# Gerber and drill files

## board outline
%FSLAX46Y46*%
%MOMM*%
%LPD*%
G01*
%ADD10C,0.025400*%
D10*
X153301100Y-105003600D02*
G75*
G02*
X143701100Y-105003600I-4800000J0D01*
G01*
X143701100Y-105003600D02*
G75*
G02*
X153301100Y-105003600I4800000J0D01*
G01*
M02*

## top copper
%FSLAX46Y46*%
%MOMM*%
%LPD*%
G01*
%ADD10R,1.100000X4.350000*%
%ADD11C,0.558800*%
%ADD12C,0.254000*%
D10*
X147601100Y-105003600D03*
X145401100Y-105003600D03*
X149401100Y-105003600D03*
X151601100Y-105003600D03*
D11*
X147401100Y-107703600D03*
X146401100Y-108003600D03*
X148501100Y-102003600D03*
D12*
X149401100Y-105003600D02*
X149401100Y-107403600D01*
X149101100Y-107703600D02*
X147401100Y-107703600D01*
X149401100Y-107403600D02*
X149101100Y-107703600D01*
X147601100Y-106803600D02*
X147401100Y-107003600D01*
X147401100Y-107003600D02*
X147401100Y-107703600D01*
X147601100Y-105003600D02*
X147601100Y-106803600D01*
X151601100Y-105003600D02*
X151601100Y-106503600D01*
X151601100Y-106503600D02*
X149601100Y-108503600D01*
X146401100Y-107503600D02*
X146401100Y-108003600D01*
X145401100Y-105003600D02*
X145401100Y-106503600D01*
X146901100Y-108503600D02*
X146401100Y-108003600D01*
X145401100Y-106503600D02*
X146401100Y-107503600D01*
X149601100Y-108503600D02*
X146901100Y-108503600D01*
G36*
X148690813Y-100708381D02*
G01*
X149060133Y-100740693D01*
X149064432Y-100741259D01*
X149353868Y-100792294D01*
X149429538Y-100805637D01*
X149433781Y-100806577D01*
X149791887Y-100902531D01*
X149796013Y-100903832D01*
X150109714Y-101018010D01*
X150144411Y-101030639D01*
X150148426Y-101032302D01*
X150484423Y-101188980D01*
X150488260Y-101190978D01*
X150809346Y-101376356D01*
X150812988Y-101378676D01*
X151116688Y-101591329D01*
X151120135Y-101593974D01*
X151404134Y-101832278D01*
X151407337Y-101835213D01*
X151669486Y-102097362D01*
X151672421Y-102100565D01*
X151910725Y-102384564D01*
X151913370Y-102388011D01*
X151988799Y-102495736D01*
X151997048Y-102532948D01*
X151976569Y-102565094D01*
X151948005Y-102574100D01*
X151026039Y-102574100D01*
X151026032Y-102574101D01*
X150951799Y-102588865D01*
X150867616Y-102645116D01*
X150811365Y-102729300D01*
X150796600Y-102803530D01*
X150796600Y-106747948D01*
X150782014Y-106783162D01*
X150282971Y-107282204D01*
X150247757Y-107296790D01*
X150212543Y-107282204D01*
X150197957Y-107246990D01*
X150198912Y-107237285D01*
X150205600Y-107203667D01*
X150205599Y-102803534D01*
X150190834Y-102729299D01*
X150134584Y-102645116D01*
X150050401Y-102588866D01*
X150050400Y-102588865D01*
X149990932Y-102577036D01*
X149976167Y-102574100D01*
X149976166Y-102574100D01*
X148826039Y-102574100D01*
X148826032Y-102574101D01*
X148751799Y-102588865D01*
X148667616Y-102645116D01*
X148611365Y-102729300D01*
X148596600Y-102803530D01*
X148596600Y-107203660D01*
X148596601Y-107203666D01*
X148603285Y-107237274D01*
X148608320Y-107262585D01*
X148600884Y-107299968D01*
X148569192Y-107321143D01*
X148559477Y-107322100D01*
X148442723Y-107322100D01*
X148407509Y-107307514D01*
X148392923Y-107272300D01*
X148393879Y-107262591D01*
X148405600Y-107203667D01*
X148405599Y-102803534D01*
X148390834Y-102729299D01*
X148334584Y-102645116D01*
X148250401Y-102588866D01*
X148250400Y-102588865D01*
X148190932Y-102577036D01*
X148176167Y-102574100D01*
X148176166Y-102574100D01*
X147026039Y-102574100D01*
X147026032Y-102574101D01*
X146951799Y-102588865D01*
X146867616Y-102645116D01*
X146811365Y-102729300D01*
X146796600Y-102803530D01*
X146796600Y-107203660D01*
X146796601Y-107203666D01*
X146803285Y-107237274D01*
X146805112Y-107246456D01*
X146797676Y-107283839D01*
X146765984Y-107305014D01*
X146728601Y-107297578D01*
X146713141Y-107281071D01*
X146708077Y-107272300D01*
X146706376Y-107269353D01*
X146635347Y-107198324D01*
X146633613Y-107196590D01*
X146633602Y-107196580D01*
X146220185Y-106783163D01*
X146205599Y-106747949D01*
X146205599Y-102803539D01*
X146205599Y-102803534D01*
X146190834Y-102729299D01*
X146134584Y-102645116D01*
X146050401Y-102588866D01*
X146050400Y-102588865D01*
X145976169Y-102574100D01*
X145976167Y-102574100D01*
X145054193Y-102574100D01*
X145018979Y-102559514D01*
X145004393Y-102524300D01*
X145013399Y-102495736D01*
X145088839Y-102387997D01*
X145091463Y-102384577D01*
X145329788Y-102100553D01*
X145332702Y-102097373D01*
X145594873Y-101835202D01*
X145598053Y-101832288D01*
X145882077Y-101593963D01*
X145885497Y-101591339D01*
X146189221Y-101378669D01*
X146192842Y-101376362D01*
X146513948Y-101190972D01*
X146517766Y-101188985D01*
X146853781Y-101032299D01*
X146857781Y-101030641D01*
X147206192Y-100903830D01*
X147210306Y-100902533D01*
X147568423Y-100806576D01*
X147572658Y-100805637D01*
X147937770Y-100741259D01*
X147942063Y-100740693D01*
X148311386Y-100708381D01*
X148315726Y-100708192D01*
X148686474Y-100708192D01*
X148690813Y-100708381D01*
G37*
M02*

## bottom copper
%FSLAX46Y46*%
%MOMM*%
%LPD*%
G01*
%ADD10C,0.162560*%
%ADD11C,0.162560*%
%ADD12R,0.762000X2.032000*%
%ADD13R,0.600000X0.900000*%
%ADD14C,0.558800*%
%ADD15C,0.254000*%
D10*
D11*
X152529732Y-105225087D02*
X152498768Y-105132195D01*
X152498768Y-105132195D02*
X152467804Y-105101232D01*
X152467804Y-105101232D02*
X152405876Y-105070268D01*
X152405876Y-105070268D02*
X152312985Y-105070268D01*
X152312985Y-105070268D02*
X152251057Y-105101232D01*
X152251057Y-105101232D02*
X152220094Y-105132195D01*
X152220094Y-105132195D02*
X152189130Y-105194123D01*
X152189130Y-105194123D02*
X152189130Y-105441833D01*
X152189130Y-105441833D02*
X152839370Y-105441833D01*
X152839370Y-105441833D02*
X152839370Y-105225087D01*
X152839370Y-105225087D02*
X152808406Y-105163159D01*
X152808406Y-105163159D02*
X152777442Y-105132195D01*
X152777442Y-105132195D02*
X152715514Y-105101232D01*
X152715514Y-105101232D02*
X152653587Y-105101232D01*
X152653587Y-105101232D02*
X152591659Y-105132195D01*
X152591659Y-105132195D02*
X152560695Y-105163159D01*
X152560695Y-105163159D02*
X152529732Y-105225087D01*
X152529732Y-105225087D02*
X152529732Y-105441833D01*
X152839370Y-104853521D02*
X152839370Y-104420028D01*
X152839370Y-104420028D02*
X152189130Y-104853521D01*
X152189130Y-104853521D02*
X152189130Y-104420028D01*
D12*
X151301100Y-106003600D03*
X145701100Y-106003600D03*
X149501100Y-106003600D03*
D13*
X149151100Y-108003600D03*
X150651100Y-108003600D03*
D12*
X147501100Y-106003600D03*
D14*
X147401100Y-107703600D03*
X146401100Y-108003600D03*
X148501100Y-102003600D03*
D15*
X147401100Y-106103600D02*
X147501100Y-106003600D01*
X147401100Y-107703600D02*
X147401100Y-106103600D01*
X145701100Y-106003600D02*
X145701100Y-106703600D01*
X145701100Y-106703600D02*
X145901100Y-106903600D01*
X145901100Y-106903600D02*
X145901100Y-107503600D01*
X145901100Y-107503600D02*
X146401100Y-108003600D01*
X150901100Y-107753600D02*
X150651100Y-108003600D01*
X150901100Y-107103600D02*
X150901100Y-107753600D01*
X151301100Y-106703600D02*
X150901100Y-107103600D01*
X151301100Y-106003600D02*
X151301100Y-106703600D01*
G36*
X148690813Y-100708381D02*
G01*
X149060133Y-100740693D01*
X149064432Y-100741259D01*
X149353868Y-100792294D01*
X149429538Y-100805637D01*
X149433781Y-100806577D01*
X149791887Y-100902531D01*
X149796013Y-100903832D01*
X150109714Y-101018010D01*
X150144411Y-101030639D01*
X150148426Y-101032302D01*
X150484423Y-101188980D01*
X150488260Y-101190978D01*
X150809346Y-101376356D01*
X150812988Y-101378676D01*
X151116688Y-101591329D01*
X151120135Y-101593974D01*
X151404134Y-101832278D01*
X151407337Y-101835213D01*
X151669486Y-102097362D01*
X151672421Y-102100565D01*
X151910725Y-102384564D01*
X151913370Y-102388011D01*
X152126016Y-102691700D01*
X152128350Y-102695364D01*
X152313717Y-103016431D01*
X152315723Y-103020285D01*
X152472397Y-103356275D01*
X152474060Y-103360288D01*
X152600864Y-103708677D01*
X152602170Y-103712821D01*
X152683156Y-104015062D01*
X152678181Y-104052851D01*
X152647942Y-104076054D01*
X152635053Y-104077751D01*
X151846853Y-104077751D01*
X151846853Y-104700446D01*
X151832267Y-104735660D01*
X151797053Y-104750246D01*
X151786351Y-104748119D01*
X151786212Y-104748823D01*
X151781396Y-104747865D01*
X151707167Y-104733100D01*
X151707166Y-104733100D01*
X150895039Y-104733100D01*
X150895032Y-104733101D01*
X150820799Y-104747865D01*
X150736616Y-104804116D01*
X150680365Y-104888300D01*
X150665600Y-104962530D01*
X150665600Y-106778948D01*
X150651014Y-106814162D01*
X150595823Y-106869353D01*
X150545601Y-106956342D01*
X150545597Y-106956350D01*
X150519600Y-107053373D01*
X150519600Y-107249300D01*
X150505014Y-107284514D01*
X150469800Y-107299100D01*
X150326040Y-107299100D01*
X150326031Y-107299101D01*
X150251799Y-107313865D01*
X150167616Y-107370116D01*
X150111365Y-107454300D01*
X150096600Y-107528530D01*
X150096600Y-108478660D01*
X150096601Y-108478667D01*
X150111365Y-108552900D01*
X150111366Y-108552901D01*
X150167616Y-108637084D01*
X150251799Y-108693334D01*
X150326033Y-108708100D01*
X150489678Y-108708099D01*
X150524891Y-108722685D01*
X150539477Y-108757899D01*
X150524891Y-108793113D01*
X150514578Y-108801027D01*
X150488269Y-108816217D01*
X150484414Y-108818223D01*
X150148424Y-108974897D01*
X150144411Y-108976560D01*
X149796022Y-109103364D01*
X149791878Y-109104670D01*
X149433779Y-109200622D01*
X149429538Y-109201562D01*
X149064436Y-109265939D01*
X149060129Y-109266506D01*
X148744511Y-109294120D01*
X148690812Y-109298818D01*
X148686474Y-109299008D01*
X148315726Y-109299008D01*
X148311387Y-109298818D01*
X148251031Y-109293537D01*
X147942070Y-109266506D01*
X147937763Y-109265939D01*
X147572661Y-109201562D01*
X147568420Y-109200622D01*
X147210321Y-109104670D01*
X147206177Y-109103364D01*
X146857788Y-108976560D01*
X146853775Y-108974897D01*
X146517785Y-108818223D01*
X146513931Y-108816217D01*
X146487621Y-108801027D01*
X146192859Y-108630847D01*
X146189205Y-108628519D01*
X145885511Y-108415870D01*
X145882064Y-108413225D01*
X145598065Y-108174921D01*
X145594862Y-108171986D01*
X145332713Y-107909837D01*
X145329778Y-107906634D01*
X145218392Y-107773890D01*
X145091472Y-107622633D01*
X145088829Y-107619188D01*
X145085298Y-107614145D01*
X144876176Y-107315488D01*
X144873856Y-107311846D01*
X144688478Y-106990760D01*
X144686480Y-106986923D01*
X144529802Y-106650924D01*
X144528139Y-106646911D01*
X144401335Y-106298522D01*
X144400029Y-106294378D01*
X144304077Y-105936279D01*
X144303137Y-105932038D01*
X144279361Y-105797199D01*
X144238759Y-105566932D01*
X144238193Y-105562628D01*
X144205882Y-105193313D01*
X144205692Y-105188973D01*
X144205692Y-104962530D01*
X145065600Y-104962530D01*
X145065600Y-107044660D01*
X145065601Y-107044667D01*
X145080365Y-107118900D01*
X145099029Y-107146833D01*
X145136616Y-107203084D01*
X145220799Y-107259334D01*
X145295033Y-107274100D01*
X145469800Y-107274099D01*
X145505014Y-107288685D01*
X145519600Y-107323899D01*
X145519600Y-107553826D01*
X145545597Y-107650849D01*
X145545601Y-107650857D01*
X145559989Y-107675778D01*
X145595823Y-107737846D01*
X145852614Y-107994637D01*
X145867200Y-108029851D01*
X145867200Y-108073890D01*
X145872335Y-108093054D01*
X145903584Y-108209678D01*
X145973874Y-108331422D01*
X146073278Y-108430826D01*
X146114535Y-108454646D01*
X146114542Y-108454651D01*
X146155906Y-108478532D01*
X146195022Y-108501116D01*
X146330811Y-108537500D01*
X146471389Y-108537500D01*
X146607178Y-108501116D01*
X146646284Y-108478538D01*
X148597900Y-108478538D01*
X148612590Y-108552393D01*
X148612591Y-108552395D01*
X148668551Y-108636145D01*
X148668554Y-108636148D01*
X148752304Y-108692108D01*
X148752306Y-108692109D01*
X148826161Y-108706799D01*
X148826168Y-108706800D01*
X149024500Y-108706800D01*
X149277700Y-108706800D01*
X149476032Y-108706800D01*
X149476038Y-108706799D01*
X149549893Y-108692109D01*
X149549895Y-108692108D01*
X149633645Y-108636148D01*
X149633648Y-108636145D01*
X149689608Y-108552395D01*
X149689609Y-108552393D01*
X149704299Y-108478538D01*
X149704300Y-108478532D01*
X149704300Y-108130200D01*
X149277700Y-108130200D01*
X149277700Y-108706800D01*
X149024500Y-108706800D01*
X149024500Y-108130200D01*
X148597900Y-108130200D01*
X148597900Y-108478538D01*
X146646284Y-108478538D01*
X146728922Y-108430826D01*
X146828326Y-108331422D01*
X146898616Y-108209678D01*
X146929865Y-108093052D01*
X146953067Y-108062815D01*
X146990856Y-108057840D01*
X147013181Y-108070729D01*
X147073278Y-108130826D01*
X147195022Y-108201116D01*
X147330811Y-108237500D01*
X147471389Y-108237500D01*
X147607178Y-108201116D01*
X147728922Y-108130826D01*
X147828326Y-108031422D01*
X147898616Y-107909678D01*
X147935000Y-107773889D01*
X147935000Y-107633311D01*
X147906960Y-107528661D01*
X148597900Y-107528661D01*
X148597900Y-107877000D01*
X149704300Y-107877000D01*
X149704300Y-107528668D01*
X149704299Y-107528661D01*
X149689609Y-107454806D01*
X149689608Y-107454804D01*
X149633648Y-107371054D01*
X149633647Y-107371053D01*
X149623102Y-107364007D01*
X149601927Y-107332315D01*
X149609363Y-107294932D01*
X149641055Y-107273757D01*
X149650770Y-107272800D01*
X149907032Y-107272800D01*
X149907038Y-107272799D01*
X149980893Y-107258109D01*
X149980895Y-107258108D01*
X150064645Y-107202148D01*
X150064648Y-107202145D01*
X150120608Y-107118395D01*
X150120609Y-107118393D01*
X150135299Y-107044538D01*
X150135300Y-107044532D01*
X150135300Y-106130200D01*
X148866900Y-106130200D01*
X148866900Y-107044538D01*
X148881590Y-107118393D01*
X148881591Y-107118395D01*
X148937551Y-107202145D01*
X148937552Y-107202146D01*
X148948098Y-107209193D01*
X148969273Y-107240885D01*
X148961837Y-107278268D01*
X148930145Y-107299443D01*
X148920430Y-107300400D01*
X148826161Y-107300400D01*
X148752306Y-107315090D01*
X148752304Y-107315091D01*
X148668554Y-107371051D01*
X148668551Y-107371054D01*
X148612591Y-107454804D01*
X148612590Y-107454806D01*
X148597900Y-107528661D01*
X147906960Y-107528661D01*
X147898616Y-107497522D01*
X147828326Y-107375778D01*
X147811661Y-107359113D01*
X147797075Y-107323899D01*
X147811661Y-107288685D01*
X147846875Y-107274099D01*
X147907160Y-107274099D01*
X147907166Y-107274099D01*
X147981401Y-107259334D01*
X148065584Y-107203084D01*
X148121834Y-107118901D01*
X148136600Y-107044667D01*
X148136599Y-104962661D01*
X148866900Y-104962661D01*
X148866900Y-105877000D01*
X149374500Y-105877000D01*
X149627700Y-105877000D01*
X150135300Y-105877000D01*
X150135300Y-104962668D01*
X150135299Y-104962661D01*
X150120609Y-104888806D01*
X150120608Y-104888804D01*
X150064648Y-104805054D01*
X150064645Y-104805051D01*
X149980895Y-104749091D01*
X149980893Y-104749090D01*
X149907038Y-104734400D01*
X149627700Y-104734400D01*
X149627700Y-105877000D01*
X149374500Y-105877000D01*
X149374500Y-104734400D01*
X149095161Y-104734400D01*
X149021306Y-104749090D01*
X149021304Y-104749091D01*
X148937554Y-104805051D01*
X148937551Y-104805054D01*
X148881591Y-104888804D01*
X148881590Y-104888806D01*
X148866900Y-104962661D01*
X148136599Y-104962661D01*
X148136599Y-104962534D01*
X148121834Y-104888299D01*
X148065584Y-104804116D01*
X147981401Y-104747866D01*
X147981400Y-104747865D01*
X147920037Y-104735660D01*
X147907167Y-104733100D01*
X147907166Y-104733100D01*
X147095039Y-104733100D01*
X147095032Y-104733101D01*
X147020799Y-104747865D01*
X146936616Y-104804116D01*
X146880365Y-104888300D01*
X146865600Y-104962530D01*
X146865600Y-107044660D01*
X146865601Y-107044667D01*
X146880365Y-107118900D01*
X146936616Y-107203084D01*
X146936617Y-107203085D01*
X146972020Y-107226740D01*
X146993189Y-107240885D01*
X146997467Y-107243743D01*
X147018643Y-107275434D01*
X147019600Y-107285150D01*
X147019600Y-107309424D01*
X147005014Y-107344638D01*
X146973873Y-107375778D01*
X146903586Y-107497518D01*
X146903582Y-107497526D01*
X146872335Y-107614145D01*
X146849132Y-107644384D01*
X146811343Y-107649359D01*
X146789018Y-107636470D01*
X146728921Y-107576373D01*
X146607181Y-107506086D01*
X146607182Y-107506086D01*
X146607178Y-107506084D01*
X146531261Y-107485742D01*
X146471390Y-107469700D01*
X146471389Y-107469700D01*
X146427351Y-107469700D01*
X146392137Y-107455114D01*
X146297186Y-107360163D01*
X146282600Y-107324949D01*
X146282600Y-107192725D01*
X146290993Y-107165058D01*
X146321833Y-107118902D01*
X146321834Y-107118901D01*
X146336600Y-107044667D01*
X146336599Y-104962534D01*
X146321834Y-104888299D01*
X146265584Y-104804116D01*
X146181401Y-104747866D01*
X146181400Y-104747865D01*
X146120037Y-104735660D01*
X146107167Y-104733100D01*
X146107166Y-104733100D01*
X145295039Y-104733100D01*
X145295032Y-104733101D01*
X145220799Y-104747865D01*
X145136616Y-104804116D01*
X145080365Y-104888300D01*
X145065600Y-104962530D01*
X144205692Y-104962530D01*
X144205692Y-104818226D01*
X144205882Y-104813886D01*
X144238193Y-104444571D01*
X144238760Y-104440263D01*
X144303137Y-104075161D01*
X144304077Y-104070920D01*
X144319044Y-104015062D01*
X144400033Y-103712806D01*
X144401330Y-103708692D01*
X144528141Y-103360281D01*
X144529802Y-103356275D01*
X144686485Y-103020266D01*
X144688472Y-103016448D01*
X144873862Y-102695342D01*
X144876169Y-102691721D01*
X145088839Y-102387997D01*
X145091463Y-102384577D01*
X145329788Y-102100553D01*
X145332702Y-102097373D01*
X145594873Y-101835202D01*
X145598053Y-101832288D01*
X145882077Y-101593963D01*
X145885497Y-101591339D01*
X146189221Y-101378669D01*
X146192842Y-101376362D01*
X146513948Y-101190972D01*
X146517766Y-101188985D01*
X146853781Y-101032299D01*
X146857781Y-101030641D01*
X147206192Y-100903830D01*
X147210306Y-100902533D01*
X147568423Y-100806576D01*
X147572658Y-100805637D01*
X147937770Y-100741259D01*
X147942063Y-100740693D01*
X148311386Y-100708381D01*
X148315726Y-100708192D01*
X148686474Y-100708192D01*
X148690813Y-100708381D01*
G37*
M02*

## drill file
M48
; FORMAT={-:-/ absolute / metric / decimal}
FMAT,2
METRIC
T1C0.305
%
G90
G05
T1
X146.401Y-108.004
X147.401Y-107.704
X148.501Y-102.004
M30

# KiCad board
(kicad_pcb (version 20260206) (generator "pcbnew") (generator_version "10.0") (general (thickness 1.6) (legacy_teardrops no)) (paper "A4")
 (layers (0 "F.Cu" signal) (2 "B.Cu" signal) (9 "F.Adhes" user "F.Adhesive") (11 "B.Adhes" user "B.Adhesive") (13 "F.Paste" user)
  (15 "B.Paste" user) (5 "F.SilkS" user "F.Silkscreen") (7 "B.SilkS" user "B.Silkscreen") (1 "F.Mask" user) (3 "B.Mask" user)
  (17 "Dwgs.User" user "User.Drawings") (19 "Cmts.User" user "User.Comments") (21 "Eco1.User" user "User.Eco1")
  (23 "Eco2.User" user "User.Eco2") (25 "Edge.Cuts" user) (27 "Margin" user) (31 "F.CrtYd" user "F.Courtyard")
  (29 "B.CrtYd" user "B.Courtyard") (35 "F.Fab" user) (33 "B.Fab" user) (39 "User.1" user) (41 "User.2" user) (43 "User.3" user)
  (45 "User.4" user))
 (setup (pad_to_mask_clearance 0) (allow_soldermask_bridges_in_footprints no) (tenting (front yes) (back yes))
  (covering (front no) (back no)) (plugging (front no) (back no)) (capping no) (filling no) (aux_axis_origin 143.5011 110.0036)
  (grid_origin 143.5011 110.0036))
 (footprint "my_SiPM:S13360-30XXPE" (layer "F.Cu") (at 146.5011 105.0036 -90)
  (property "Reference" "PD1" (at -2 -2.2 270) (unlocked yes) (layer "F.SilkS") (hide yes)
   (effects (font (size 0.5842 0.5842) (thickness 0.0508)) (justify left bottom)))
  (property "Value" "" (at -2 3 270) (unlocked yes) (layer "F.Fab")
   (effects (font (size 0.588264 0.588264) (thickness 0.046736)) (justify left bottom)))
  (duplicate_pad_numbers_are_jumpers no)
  (pad "A" smd rect (at 0 -1.1 270) (size 4.35 1.1) (layers "F.Cu" "F.Mask" "F.Paste") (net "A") (solder_mask_margin 0.0635)
   (solder_paste_margin 0) (thermal_bridge_angle 0))
  (pad "C" smd rect (at 0 1.1 270) (size 4.35 1.1) (layers "F.Cu" "F.Mask" "F.Paste") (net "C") (solder_mask_margin 0.0635)
   (solder_paste_margin 0) (thermal_bridge_angle 0)))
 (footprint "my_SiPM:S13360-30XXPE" (layer "F.Cu") (at 150.5011 105.0036 90)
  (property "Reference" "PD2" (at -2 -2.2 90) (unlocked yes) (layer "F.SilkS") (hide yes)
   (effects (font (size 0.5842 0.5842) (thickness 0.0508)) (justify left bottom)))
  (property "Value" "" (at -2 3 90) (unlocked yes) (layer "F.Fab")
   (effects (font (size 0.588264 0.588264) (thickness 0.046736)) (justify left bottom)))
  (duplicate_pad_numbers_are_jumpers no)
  (pad "A" smd rect (at 0 -1.1 90) (size 4.35 1.1) (layers "F.Cu" "F.Mask" "F.Paste") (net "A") (solder_mask_margin 0.0635)
   (solder_paste_margin 0) (thermal_bridge_angle 0))
  (pad "C" smd rect (at 0 1.1 90) (size 4.35 1.1) (layers "F.Cu" "F.Mask" "F.Paste") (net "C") (solder_mask_margin 0.0635)
   (solder_paste_margin 0) (thermal_bridge_angle 0)))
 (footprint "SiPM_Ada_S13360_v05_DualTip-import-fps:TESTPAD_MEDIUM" (layer "B.Cu") (at 151.3011 106.0036 -90)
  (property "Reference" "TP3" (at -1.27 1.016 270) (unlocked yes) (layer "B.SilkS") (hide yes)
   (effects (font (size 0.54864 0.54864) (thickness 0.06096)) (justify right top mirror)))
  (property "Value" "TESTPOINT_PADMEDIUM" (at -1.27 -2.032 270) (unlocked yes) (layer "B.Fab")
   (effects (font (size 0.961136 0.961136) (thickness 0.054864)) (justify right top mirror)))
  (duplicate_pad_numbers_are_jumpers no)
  (pad "P$1" smd rect (at 0 0 270) (size 2.032 0.762) (layers "B.Cu" "B.Mask") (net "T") (solder_mask_margin 0.0635) (solder_paste_margin 0)
   (thermal_bridge_angle 0)))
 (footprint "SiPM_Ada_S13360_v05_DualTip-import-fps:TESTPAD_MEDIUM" (layer "B.Cu") (at 145.7011 106.0036 -90)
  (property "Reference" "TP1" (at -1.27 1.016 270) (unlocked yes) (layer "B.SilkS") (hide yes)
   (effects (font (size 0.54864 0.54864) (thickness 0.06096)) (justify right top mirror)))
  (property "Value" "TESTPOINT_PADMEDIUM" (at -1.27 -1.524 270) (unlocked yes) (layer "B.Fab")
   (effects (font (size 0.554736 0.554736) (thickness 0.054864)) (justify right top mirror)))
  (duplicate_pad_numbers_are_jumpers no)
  (pad "P$1" smd rect (at 0 0 270) (size 2.032 0.762) (layers "B.Cu" "B.Mask") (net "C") (solder_mask_margin 0.0635) (solder_paste_margin 0)
   (thermal_bridge_angle 0)))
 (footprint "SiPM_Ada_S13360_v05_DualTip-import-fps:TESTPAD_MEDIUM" (layer "B.Cu") (at 149.5011 106.0036 -90)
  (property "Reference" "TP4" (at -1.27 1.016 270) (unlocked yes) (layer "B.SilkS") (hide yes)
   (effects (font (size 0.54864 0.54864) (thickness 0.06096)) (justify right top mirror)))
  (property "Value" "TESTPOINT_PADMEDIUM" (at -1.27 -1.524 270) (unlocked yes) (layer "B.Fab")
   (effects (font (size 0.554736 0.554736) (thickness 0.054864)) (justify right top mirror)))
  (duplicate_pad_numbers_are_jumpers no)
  (pad "P$1" smd rect (at 0 0 270) (size 2.032 0.762) (layers "B.Cu" "B.Mask") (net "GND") (solder_mask_margin 0.0635)
   (solder_paste_margin 0) (thermal_bridge_angle 0)))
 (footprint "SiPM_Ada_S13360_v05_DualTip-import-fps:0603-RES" (layer "B.Cu") (at 149.9011 108.0036)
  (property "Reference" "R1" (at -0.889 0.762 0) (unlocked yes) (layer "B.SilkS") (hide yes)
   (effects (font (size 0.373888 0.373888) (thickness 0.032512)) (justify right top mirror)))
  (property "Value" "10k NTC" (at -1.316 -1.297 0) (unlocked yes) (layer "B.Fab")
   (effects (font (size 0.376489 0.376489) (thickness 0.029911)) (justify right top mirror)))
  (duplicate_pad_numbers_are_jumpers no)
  (pad "1" smd rect (at -0.75 0) (size 0.6 0.9) (layers "B.Cu" "B.Mask" "B.Paste") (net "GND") (solder_mask_margin 0.0635)
   (solder_paste_margin 0) (thermal_bridge_angle 0))
  (pad "2" smd rect (at 0.75 0) (size 0.6 0.9) (layers "B.Cu" "B.Mask" "B.Paste") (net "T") (solder_mask_margin 0.0635)
   (solder_paste_margin 0) (thermal_bridge_angle 0)))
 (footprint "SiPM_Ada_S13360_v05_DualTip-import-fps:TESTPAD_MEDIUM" (layer "B.Cu") (at 147.5011 106.0036 -90)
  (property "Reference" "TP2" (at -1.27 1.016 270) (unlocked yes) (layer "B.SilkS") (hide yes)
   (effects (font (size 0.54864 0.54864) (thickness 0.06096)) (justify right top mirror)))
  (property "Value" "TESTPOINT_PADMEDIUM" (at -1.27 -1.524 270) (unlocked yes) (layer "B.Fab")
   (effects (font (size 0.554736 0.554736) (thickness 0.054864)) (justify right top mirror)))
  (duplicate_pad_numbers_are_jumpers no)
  (pad "P$1" smd rect (at 0 0 270) (size 2.032 0.762) (layers "B.Cu" "B.Mask") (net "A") (solder_mask_margin 0.0635) (solder_paste_margin 0)
   (thermal_bridge_angle 0)))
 (gr_circle (center 148.5011 105.0036) (end 153.3011 105.0036) (stroke (width 0.0254) (type solid)) (fill no) (layer "Edge.Cuts"))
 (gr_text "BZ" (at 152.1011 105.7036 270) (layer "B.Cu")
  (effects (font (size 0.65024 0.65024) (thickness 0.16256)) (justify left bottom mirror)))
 (segment (start 149.4011 105.0036) (end 149.4011 107.4036) (width 0.254) (layer "F.Cu") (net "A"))
 (segment (start 149.1011 107.7036) (end 147.4011 107.7036) (width 0.254) (layer "F.Cu") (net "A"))
 (segment (start 149.4011 107.4036) (end 149.1011 107.7036) (width 0.254) (layer "F.Cu") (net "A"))
 (segment (start 147.6011 106.8036) (end 147.4011 107.0036) (width 0.254) (layer "F.Cu") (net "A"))
 (segment (start 147.4011 107.0036) (end 147.4011 107.7036) (width 0.254) (layer "F.Cu") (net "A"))
 (segment (start 147.6011 105.0036) (end 147.6011 106.8036) (width 0.254) (layer "F.Cu") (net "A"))
 (via (at 147.4011 107.7036) (size 0.5588) (drill 0.3048) (layers "F.Cu" "B.Cu") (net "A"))
 (segment (start 147.4011 106.1036) (end 147.5011 106.0036) (width 0.254) (layer "B.Cu") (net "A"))
 (segment (start 147.4011 107.7036) (end 147.4011 106.1036) (width 0.254) (layer "B.Cu") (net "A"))
 (segment (start 151.6011 105.0036) (end 151.6011 106.5036) (width 0.254) (layer "F.Cu") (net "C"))
 (segment (start 151.6011 106.5036) (end 149.6011 108.5036) (width 0.254) (layer "F.Cu") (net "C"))
 (segment (start 146.4011 107.5036) (end 146.4011 108.0036) (width 0.254) (layer "F.Cu") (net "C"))
 (segment (start 145.4011 105.0036) (end 145.4011 106.5036) (width 0.254) (layer "F.Cu") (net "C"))
 (segment (start 146.9011 108.5036) (end 146.4011 108.0036) (width 0.254) (layer "F.Cu") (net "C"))
 (segment (start 145.4011 106.5036) (end 146.4011 107.5036) (width 0.254) (layer "F.Cu") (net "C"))
 (segment (start 149.6011 108.5036) (end 146.9011 108.5036) (width 0.254) (layer "F.Cu") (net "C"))
 (via (at 146.4011 108.0036) (size 0.5588) (drill 0.3048) (layers "F.Cu" "B.Cu") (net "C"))
 (segment (start 145.7011 106.0036) (end 145.7011 106.7036) (width 0.254) (layer "B.Cu") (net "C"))
 (segment (start 145.7011 106.7036) (end 145.9011 106.9036) (width 0.254) (layer "B.Cu") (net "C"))
 (segment (start 145.9011 106.9036) (end 145.9011 107.5036) (width 0.254) (layer "B.Cu") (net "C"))
 (segment (start 145.9011 107.5036) (end 146.4011 108.0036) (width 0.254) (layer "B.Cu") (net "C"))
 (segment (start 150.9011 107.7536) (end 150.6511 108.0036) (width 0.254) (layer "B.Cu") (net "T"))
 (segment (start 150.9011 107.1036) (end 150.9011 107.7536) (width 0.254) (layer "B.Cu") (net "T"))
 (segment (start 151.3011 106.7036) (end 150.9011 107.1036) (width 0.254) (layer "B.Cu") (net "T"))
 (segment (start 151.3011 106.0036) (end 151.3011 106.7036) (width 0.254) (layer "B.Cu") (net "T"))
 (via (at 148.5011 102.0036) (size 0.5588) (drill 0.3048) (layers "F.Cu" "B.Cu") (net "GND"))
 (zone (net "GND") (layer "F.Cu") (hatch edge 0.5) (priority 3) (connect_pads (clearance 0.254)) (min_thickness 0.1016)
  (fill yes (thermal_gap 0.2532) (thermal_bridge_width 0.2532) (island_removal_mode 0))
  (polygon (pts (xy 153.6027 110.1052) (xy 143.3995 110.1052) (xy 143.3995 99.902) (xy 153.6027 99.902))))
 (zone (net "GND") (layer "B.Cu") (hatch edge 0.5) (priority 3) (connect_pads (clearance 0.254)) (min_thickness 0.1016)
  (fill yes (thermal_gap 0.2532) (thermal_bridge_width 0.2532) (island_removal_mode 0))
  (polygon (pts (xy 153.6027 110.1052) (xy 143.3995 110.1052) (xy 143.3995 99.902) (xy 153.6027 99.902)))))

